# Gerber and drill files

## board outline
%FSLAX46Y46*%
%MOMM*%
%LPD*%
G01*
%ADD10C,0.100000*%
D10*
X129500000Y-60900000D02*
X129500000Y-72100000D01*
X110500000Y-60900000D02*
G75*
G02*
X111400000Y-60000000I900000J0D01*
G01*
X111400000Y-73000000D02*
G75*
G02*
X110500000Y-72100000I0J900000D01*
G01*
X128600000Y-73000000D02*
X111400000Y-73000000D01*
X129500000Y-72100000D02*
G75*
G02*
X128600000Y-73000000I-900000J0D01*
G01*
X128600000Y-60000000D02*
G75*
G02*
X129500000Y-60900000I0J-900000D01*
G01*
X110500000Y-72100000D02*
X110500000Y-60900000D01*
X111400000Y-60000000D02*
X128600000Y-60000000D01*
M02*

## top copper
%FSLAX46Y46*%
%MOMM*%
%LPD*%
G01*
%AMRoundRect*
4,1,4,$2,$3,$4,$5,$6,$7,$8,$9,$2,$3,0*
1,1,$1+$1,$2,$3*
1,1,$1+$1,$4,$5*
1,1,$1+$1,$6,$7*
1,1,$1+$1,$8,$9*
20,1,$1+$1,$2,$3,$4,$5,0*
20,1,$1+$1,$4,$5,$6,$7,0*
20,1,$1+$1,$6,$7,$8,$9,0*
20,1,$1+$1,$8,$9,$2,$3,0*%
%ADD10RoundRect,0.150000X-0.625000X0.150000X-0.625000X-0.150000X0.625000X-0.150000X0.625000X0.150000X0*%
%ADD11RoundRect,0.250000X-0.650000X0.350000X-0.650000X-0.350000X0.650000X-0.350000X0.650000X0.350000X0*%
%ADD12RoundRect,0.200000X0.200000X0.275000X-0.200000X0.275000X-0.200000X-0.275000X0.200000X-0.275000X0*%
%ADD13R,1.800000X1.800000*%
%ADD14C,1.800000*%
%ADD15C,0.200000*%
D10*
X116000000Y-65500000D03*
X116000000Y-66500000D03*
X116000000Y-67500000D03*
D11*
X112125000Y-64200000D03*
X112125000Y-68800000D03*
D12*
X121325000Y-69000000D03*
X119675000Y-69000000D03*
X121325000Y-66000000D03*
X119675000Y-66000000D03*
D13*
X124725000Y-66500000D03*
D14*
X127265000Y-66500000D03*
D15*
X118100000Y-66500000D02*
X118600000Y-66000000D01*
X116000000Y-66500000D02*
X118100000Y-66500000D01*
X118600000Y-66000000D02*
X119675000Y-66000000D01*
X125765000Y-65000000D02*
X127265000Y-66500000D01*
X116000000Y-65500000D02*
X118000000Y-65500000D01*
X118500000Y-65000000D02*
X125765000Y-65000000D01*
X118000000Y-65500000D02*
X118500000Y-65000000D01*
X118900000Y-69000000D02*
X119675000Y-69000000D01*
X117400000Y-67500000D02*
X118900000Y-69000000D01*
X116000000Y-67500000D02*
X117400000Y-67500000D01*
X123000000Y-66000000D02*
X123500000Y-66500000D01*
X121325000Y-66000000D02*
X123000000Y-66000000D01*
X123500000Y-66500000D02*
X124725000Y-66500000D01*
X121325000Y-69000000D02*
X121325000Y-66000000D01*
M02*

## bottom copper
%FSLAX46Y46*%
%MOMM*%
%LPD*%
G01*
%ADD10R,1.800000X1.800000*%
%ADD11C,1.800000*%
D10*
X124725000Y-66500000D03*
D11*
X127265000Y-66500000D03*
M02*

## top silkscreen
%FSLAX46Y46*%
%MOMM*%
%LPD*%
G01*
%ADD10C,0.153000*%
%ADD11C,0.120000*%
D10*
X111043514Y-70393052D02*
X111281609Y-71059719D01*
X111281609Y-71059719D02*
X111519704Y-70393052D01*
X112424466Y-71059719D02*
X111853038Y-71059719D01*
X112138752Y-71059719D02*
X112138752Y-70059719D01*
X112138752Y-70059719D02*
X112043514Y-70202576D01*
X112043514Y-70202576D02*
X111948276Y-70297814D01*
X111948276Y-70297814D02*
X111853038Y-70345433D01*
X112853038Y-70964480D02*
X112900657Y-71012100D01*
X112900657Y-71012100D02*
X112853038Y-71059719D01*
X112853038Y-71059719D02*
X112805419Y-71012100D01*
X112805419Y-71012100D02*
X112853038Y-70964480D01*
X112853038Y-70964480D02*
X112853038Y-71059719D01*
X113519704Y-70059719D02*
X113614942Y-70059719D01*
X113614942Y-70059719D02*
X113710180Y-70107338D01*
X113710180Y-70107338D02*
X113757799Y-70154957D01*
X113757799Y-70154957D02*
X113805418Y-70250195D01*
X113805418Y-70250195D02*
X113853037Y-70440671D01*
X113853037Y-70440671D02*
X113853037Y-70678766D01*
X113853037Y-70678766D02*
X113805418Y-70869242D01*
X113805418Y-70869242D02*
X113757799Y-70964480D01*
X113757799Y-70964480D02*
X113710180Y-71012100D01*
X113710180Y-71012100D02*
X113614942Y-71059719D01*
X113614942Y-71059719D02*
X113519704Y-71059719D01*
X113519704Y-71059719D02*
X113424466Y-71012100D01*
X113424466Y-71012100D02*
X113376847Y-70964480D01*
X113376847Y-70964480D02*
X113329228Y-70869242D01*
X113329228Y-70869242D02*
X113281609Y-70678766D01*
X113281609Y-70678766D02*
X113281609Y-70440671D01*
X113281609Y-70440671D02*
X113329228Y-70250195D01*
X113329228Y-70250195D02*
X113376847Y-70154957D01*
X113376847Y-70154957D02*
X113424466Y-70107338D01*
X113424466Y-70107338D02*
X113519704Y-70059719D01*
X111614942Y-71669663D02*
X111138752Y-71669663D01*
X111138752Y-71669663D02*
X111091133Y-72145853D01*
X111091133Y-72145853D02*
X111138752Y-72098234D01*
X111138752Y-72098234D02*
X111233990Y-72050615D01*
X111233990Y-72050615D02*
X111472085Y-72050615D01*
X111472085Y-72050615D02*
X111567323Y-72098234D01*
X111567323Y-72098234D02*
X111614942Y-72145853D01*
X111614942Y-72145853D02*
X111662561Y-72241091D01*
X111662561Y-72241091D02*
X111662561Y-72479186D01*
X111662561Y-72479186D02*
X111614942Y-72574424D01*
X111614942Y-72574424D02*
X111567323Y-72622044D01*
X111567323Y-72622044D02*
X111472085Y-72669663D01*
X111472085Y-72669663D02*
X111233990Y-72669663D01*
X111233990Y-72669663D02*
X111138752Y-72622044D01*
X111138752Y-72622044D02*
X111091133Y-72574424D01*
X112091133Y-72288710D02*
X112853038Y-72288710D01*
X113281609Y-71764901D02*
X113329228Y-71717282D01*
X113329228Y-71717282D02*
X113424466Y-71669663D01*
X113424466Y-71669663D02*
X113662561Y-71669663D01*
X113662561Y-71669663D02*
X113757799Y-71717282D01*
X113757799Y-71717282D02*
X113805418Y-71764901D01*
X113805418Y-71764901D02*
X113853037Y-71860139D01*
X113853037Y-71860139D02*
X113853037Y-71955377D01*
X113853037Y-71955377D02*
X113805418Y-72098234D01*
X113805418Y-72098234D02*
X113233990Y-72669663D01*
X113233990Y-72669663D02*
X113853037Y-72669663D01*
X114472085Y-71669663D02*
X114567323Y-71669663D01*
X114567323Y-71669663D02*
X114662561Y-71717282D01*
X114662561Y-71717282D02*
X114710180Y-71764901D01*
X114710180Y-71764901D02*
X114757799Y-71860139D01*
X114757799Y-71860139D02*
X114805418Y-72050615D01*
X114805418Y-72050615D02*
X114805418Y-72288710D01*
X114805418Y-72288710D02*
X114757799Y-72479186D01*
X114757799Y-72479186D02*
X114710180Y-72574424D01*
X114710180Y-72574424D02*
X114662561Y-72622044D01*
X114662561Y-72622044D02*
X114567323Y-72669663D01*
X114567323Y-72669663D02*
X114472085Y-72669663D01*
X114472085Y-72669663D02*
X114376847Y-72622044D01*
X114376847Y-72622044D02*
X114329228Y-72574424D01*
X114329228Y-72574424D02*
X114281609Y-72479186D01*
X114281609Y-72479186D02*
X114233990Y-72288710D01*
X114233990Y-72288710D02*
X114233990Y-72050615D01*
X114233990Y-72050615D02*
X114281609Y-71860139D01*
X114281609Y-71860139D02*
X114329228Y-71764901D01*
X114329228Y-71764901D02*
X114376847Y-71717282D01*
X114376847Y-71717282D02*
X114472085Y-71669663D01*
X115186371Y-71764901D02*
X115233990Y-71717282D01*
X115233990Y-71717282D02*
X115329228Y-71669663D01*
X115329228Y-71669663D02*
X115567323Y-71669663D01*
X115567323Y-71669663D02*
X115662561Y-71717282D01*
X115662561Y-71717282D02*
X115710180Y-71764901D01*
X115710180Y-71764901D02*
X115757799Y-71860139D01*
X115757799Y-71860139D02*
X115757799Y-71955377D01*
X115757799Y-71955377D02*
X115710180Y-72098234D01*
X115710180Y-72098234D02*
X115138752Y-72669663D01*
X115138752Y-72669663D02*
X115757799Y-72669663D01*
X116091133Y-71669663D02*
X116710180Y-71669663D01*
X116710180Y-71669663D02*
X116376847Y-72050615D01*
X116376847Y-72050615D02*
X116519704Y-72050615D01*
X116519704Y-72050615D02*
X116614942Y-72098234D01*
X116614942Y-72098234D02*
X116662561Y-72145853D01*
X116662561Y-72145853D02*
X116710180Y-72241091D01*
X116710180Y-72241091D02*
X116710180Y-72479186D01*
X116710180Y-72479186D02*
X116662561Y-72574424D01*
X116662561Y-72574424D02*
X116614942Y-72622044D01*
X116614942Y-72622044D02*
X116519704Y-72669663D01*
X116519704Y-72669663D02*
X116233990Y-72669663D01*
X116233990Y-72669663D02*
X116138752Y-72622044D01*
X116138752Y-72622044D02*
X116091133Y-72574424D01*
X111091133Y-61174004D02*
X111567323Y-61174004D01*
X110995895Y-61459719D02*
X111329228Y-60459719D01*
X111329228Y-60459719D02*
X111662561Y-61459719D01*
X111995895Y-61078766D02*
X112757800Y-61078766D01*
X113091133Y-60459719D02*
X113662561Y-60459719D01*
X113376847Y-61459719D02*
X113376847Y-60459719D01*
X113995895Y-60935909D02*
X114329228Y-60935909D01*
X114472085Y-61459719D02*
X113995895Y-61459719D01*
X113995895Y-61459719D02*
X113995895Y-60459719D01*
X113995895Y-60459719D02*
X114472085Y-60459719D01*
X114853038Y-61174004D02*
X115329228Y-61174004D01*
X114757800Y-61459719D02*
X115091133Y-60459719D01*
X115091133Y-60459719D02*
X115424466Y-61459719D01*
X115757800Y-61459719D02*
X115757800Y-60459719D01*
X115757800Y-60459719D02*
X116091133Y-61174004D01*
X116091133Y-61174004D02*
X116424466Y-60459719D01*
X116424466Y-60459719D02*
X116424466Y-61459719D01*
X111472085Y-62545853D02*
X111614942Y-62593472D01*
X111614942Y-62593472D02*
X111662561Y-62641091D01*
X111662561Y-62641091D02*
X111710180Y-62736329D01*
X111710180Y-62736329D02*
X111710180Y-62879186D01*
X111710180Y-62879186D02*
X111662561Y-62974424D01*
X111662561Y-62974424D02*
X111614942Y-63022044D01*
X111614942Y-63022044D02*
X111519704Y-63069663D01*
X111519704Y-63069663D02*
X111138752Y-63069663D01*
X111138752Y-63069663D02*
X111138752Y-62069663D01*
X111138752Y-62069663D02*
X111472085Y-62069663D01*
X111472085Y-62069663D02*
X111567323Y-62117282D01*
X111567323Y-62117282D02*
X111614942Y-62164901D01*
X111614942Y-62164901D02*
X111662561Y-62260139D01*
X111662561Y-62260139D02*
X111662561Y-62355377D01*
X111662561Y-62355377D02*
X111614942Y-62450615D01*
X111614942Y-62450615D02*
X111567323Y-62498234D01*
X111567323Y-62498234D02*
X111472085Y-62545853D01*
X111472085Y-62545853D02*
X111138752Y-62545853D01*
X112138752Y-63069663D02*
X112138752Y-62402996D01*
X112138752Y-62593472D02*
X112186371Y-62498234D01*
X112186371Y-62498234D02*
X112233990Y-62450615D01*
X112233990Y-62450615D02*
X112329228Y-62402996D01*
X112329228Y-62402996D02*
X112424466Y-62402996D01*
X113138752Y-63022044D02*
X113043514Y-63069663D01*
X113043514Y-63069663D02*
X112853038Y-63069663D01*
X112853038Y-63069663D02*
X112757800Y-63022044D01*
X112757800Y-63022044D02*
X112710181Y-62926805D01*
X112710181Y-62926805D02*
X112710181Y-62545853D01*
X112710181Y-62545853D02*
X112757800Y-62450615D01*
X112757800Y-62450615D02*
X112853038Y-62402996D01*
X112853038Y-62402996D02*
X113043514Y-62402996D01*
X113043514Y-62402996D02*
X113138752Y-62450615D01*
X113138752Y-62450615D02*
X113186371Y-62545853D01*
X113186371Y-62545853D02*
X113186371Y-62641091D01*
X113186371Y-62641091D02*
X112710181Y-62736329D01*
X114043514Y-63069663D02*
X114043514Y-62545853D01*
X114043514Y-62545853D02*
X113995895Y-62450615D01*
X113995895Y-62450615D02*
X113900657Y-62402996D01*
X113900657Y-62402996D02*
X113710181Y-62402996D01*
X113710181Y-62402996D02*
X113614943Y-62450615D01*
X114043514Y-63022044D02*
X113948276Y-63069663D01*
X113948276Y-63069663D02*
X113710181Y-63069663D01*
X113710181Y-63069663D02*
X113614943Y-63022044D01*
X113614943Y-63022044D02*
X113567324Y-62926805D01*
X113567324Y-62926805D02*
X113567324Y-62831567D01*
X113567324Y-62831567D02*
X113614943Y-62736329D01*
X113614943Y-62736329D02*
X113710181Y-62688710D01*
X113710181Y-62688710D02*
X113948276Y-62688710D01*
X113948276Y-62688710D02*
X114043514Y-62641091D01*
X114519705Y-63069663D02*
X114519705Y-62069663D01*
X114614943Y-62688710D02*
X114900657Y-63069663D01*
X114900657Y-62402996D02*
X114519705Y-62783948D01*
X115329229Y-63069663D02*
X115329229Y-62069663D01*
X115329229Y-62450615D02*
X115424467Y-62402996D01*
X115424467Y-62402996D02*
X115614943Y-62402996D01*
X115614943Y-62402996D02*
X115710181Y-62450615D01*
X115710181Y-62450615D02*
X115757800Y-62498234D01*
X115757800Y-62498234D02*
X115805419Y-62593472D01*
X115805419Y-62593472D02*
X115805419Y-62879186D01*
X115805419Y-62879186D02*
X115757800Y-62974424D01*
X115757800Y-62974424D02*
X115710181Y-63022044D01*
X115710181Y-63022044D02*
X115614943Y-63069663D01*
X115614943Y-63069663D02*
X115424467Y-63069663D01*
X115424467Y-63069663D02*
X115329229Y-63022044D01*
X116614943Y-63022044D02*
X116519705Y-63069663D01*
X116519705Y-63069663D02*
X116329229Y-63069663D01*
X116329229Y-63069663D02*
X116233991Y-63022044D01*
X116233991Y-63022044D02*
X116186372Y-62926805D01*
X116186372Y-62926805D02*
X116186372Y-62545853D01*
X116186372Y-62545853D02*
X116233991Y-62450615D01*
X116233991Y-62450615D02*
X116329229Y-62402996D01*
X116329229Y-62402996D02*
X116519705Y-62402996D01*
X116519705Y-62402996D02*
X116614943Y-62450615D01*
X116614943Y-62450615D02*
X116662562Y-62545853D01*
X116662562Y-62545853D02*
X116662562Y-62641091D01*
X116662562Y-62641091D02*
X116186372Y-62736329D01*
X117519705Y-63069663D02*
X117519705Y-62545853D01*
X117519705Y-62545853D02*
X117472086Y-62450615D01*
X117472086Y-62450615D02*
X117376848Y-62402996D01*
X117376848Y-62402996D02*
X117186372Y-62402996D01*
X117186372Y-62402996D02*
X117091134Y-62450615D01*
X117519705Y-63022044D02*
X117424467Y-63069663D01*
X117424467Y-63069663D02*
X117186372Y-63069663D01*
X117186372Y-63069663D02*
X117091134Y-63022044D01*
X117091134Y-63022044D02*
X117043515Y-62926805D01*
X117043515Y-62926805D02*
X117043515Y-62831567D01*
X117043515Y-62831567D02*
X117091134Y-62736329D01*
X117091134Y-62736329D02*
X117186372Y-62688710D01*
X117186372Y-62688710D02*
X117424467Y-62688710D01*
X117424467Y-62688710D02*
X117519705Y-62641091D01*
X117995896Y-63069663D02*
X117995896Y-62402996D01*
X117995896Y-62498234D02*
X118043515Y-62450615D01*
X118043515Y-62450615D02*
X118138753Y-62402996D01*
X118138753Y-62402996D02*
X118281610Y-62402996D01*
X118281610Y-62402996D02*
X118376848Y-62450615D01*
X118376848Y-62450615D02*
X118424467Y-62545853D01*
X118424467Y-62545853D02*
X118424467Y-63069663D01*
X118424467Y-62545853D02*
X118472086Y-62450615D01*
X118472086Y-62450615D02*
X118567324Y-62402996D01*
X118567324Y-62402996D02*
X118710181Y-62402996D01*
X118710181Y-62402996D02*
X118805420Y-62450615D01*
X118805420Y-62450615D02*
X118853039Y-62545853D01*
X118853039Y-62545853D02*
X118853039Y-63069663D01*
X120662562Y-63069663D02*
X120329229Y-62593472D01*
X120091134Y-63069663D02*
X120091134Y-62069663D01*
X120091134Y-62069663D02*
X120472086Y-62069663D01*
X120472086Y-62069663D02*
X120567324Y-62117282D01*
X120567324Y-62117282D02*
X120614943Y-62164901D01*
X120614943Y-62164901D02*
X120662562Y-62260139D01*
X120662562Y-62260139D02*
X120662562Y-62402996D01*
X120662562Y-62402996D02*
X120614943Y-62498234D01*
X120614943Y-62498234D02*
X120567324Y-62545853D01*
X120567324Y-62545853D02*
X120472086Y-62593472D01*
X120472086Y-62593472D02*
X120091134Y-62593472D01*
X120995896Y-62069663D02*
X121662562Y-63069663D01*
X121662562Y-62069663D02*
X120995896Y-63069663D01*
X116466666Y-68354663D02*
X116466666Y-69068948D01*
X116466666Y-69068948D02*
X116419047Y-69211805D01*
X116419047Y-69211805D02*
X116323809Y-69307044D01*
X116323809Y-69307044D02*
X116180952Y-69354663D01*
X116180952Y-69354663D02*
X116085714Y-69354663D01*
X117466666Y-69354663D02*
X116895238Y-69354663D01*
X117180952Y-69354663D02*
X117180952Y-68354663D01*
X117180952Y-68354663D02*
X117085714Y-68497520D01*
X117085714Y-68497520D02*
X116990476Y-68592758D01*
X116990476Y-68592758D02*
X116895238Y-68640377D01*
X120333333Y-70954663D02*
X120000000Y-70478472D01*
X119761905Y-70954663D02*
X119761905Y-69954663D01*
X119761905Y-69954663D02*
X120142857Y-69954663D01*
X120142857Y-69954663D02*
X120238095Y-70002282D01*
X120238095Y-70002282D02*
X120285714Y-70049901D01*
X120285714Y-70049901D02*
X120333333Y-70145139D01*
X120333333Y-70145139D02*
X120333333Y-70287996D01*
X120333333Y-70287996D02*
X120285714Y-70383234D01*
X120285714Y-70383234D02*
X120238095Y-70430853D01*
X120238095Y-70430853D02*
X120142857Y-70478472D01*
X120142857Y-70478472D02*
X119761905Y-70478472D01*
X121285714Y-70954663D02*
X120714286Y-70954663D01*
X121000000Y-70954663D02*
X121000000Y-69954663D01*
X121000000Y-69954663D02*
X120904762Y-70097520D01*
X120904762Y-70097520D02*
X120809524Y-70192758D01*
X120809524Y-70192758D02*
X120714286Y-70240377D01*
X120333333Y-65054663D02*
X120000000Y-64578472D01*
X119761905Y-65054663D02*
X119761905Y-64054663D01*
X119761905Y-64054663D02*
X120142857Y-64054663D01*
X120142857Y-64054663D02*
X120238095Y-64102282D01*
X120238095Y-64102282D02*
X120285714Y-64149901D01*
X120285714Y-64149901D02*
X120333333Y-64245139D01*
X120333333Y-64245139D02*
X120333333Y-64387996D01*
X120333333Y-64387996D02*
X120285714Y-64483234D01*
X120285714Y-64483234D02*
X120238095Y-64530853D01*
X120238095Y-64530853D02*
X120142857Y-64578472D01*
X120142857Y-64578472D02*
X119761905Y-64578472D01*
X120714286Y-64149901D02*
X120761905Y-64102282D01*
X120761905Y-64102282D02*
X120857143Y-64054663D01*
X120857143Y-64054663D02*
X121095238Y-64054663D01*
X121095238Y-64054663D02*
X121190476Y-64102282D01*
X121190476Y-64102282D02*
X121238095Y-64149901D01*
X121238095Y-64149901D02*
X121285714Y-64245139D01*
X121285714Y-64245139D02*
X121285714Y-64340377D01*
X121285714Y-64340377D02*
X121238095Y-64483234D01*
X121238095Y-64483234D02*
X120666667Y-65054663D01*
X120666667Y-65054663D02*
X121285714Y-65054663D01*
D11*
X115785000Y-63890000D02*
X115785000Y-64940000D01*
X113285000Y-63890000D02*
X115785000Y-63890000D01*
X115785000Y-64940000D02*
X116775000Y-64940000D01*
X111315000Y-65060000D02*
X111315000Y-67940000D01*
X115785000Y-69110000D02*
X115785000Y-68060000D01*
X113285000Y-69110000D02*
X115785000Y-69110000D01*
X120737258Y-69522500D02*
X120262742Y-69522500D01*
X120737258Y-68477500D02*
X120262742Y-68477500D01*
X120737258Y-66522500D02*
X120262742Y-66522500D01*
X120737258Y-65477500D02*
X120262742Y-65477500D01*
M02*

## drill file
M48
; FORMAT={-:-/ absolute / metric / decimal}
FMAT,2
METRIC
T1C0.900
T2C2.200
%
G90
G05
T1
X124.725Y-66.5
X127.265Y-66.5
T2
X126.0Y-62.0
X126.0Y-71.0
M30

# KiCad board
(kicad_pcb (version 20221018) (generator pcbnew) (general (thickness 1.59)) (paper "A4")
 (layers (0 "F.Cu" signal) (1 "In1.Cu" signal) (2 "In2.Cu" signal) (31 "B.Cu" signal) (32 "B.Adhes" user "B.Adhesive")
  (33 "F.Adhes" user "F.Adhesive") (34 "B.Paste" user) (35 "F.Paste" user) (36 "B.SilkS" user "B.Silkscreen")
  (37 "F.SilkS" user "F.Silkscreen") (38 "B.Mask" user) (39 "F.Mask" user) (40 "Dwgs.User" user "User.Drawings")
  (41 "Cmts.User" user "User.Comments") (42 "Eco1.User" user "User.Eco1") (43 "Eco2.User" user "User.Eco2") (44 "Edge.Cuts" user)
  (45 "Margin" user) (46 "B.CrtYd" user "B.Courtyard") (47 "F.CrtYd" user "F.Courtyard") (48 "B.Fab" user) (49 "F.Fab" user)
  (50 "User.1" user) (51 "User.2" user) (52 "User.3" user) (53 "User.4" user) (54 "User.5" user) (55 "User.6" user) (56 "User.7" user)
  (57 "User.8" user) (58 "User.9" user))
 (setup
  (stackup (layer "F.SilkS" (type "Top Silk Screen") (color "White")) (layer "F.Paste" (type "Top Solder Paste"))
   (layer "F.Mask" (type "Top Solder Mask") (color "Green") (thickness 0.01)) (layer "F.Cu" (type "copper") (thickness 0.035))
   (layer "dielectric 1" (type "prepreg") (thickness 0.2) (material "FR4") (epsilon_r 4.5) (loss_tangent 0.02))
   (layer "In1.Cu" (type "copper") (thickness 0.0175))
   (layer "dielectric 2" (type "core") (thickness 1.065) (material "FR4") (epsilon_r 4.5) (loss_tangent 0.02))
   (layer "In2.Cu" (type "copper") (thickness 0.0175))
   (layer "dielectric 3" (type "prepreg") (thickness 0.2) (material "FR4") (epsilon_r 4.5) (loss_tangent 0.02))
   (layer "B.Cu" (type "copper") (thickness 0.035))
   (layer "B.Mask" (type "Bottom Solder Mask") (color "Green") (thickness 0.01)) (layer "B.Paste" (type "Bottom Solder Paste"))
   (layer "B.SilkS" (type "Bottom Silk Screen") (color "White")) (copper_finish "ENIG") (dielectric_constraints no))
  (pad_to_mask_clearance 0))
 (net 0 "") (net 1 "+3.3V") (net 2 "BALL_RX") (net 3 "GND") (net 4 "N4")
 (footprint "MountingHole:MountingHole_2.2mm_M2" (layer "F.Cu") (at 126 71 -90)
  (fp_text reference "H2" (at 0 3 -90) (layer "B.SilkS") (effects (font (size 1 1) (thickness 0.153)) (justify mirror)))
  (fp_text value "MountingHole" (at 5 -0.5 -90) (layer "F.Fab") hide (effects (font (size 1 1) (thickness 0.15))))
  (pad "" np_thru_hole circle (at 0 0 270) (size 2.2 2.2) (drill 2.2) (layers "*.Cu" "*.Mask")))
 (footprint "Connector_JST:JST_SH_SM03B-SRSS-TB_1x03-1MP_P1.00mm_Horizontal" (layer "F.Cu") (at 114 66.5 -90)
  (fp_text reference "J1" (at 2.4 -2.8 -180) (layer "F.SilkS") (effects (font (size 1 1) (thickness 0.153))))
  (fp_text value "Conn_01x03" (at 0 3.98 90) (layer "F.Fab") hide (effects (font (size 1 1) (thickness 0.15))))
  (fp_line (start -2.61 -1.785) (end -1.56 -1.785) (stroke (width 0.12) (type solid)) (layer "F.SilkS"))
  (fp_line (start -2.61 0.715) (end -2.61 -1.785) (stroke (width 0.12) (type solid)) (layer "F.SilkS"))
  (fp_line (start -1.56 -1.785) (end -1.56 -2.775) (stroke (width 0.12) (type solid)) (layer "F.SilkS"))
  (fp_line (start -1.44 2.685) (end 1.44 2.685) (stroke (width 0.12) (type solid)) (layer "F.SilkS"))
  (fp_line (start 2.61 -1.785) (end 1.56 -1.785) (stroke (width 0.12) (type solid)) (layer "F.SilkS"))
  (fp_line (start 2.61 0.715) (end 2.61 -1.785) (stroke (width 0.12) (type solid)) (layer "F.SilkS"))
  (pad "1" smd roundrect (at -1 -2 270) (size 0.6 1.55) (layers "F.Cu" "F.Paste" "F.Mask") (roundrect_rratio 0.25) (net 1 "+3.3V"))
  (pad "2" smd roundrect (at 0 -2 270) (size 0.6 1.55) (layers "F.Cu" "F.Paste" "F.Mask") (roundrect_rratio 0.25) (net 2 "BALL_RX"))
  (pad "3" smd roundrect (at 1 -2 270) (size 0.6 1.55) (layers "F.Cu" "F.Paste" "F.Mask") (roundrect_rratio 0.25) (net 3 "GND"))
  (pad "MP" smd roundrect (at -2.3 1.875 270) (size 1.2 1.8) (layers "F.Cu" "F.Paste" "F.Mask") (roundrect_rratio 0.208333))
  (pad "MP" smd roundrect (at 2.3 1.875 270) (size 1.2 1.8) (layers "F.Cu" "F.Paste" "F.Mask") (roundrect_rratio 0.208333)))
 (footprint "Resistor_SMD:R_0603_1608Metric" (layer "F.Cu") (at 120.5 69 180)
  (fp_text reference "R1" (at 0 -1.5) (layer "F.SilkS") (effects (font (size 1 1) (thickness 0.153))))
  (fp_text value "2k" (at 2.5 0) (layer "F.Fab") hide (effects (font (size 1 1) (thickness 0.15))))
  (fp_line (start -0.237258 -0.5225) (end 0.237258 -0.5225) (stroke (width 0.12) (type solid)) (layer "F.SilkS"))
  (fp_line (start -0.237258 0.5225) (end 0.237258 0.5225) (stroke (width 0.12) (type solid)) (layer "F.SilkS"))
  (pad "1" smd roundrect (at -0.825 0 180) (size 0.8 0.95) (layers "F.Cu" "F.Paste" "F.Mask") (roundrect_rratio 0.25) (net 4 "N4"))
  (pad "2" smd roundrect (at 0.825 0 180) (size 0.8 0.95) (layers "F.Cu" "F.Paste" "F.Mask") (roundrect_rratio 0.25) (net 3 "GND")))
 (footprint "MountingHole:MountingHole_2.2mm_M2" (layer "F.Cu") (at 126 62 -90)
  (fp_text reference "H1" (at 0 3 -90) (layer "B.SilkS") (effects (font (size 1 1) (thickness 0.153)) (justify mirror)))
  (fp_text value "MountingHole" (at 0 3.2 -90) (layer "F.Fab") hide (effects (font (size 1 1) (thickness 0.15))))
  (pad "" np_thru_hole circle (at 0 0 270) (size 2.2 2.2) (drill 2.2) (layers "*.Cu" "*.Mask")))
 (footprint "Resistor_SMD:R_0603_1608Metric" (layer "F.Cu") (at 120.5 66 180)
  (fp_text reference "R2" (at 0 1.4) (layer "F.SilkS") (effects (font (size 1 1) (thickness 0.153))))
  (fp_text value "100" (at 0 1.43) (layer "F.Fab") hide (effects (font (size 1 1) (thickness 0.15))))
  (fp_line (start -0.237258 -0.5225) (end 0.237258 -0.5225) (stroke (width 0.12) (type solid)) (layer "F.SilkS"))
  (fp_line (start -0.237258 0.5225) (end 0.237258 0.5225) (stroke (width 0.12) (type solid)) (layer "F.SilkS"))
  (pad "1" smd roundrect (at -0.825 0 180) (size 0.8 0.95) (layers "F.Cu" "F.Paste" "F.Mask") (roundrect_rratio 0.25) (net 4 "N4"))
  (pad "2" smd roundrect (at 0.825 0 180) (size 0.8 0.95) (layers "F.Cu" "F.Paste" "F.Mask") (roundrect_rratio 0.25) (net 2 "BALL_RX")))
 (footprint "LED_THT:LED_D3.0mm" (layer "B.Cu") (at 124.725 66.5)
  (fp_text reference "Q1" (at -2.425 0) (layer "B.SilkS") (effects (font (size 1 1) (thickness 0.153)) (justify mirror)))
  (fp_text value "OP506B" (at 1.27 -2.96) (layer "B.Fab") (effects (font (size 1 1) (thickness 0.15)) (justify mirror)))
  (pad "1" thru_hole rect (at 0 0) (size 1.8 1.8) (drill 0.9) (layers "*.Cu" "*.Mask") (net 4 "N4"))
  (pad "2" thru_hole circle (at 2.54 0) (size 1.8 1.8) (drill 0.9) (layers "*.Cu" "*.Mask") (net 1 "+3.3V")))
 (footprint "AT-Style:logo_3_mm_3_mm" (layer "B.Cu") (at 117.7 64.8 180)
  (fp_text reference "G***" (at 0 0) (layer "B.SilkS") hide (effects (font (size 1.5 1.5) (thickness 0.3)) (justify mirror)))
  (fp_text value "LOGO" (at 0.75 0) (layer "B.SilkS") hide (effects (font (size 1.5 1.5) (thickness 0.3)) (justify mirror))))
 (gr_line (start 129.5 60.9) (end 129.5 72.1) (stroke (width 0.1) (type default)) (layer "Edge.Cuts"))
 (gr_arc (start 110.5 60.9) (mid 110.763604 60.263604) (end 111.4 60) (stroke (width 0.1) (type default)) (layer "Edge.Cuts"))
 (gr_arc (start 111.4 73) (mid 110.763604 72.736396) (end 110.5 72.1) (stroke (width 0.1) (type default)) (layer "Edge.Cuts"))
 (gr_line (start 128.6 73) (end 111.4 73) (stroke (width 0.1) (type default)) (layer "Edge.Cuts"))
 (gr_arc (start 129.5 72.1) (mid 129.236396 72.736396) (end 128.6 73) (stroke (width 0.1) (type default)) (layer "Edge.Cuts"))
 (gr_arc (start 128.6 60) (mid 129.236396 60.263604) (end 129.5 60.9) (stroke (width 0.1) (type default)) (layer "Edge.Cuts"))
 (gr_line (start 110.5 72.1) (end 110.5 60.9) (stroke (width 0.1) (type default)) (layer "Edge.Cuts"))
 (gr_line (start 111.4 60) (end 128.6 60) (stroke (width 0.1) (type default)) (layer "Edge.Cuts"))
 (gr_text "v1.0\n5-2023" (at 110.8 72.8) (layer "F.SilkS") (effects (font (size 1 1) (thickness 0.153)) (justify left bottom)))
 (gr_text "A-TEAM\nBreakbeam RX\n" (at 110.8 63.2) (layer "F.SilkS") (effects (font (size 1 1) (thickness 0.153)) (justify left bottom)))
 (segment (start 118.1 66.5) (end 118.6 66) (width 0.2) (layer "F.Cu") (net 2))
 (segment (start 116 66.5) (end 118.1 66.5) (width 0.2) (layer "F.Cu") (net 2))
 (segment (start 118.6 66) (end 119.675 66) (width 0.2) (layer "F.Cu") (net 2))
 (segment (start 125.765 65) (end 127.265 66.5) (width 0.2) (layer "F.Cu") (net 1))
 (segment (start 116 65.5) (end 118 65.5) (width 0.2) (layer "F.Cu") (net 1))
 (segment (start 118.5 65) (end 125.765 65) (width 0.2) (layer "F.Cu") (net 1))
 (segment (start 118 65.5) (end 118.5 65) (width 0.2) (layer "F.Cu") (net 1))
 (segment (start 118.9 69) (end 119.675 69) (width 0.2) (layer "F.Cu") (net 3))
 (segment (start 117.4 67.5) (end 118.9 69) (width 0.2) (layer "F.Cu") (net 3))
 (segment (start 116 67.5) (end 117.4 67.5) (width 0.2) (layer "F.Cu") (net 3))
 (segment (start 123 66) (end 123.5 66.5) (width 0.2) (layer "F.Cu") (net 4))
 (segment (start 121.325 66) (end 123 66) (width 0.2) (layer "F.Cu") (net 4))
 (segment (start 123.5 66.5) (end 124.725 66.5) (width 0.2) (layer "F.Cu") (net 4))
 (segment (start 121.325 69) (end 121.325 66) (width 0.2) (layer "F.Cu") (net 4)))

